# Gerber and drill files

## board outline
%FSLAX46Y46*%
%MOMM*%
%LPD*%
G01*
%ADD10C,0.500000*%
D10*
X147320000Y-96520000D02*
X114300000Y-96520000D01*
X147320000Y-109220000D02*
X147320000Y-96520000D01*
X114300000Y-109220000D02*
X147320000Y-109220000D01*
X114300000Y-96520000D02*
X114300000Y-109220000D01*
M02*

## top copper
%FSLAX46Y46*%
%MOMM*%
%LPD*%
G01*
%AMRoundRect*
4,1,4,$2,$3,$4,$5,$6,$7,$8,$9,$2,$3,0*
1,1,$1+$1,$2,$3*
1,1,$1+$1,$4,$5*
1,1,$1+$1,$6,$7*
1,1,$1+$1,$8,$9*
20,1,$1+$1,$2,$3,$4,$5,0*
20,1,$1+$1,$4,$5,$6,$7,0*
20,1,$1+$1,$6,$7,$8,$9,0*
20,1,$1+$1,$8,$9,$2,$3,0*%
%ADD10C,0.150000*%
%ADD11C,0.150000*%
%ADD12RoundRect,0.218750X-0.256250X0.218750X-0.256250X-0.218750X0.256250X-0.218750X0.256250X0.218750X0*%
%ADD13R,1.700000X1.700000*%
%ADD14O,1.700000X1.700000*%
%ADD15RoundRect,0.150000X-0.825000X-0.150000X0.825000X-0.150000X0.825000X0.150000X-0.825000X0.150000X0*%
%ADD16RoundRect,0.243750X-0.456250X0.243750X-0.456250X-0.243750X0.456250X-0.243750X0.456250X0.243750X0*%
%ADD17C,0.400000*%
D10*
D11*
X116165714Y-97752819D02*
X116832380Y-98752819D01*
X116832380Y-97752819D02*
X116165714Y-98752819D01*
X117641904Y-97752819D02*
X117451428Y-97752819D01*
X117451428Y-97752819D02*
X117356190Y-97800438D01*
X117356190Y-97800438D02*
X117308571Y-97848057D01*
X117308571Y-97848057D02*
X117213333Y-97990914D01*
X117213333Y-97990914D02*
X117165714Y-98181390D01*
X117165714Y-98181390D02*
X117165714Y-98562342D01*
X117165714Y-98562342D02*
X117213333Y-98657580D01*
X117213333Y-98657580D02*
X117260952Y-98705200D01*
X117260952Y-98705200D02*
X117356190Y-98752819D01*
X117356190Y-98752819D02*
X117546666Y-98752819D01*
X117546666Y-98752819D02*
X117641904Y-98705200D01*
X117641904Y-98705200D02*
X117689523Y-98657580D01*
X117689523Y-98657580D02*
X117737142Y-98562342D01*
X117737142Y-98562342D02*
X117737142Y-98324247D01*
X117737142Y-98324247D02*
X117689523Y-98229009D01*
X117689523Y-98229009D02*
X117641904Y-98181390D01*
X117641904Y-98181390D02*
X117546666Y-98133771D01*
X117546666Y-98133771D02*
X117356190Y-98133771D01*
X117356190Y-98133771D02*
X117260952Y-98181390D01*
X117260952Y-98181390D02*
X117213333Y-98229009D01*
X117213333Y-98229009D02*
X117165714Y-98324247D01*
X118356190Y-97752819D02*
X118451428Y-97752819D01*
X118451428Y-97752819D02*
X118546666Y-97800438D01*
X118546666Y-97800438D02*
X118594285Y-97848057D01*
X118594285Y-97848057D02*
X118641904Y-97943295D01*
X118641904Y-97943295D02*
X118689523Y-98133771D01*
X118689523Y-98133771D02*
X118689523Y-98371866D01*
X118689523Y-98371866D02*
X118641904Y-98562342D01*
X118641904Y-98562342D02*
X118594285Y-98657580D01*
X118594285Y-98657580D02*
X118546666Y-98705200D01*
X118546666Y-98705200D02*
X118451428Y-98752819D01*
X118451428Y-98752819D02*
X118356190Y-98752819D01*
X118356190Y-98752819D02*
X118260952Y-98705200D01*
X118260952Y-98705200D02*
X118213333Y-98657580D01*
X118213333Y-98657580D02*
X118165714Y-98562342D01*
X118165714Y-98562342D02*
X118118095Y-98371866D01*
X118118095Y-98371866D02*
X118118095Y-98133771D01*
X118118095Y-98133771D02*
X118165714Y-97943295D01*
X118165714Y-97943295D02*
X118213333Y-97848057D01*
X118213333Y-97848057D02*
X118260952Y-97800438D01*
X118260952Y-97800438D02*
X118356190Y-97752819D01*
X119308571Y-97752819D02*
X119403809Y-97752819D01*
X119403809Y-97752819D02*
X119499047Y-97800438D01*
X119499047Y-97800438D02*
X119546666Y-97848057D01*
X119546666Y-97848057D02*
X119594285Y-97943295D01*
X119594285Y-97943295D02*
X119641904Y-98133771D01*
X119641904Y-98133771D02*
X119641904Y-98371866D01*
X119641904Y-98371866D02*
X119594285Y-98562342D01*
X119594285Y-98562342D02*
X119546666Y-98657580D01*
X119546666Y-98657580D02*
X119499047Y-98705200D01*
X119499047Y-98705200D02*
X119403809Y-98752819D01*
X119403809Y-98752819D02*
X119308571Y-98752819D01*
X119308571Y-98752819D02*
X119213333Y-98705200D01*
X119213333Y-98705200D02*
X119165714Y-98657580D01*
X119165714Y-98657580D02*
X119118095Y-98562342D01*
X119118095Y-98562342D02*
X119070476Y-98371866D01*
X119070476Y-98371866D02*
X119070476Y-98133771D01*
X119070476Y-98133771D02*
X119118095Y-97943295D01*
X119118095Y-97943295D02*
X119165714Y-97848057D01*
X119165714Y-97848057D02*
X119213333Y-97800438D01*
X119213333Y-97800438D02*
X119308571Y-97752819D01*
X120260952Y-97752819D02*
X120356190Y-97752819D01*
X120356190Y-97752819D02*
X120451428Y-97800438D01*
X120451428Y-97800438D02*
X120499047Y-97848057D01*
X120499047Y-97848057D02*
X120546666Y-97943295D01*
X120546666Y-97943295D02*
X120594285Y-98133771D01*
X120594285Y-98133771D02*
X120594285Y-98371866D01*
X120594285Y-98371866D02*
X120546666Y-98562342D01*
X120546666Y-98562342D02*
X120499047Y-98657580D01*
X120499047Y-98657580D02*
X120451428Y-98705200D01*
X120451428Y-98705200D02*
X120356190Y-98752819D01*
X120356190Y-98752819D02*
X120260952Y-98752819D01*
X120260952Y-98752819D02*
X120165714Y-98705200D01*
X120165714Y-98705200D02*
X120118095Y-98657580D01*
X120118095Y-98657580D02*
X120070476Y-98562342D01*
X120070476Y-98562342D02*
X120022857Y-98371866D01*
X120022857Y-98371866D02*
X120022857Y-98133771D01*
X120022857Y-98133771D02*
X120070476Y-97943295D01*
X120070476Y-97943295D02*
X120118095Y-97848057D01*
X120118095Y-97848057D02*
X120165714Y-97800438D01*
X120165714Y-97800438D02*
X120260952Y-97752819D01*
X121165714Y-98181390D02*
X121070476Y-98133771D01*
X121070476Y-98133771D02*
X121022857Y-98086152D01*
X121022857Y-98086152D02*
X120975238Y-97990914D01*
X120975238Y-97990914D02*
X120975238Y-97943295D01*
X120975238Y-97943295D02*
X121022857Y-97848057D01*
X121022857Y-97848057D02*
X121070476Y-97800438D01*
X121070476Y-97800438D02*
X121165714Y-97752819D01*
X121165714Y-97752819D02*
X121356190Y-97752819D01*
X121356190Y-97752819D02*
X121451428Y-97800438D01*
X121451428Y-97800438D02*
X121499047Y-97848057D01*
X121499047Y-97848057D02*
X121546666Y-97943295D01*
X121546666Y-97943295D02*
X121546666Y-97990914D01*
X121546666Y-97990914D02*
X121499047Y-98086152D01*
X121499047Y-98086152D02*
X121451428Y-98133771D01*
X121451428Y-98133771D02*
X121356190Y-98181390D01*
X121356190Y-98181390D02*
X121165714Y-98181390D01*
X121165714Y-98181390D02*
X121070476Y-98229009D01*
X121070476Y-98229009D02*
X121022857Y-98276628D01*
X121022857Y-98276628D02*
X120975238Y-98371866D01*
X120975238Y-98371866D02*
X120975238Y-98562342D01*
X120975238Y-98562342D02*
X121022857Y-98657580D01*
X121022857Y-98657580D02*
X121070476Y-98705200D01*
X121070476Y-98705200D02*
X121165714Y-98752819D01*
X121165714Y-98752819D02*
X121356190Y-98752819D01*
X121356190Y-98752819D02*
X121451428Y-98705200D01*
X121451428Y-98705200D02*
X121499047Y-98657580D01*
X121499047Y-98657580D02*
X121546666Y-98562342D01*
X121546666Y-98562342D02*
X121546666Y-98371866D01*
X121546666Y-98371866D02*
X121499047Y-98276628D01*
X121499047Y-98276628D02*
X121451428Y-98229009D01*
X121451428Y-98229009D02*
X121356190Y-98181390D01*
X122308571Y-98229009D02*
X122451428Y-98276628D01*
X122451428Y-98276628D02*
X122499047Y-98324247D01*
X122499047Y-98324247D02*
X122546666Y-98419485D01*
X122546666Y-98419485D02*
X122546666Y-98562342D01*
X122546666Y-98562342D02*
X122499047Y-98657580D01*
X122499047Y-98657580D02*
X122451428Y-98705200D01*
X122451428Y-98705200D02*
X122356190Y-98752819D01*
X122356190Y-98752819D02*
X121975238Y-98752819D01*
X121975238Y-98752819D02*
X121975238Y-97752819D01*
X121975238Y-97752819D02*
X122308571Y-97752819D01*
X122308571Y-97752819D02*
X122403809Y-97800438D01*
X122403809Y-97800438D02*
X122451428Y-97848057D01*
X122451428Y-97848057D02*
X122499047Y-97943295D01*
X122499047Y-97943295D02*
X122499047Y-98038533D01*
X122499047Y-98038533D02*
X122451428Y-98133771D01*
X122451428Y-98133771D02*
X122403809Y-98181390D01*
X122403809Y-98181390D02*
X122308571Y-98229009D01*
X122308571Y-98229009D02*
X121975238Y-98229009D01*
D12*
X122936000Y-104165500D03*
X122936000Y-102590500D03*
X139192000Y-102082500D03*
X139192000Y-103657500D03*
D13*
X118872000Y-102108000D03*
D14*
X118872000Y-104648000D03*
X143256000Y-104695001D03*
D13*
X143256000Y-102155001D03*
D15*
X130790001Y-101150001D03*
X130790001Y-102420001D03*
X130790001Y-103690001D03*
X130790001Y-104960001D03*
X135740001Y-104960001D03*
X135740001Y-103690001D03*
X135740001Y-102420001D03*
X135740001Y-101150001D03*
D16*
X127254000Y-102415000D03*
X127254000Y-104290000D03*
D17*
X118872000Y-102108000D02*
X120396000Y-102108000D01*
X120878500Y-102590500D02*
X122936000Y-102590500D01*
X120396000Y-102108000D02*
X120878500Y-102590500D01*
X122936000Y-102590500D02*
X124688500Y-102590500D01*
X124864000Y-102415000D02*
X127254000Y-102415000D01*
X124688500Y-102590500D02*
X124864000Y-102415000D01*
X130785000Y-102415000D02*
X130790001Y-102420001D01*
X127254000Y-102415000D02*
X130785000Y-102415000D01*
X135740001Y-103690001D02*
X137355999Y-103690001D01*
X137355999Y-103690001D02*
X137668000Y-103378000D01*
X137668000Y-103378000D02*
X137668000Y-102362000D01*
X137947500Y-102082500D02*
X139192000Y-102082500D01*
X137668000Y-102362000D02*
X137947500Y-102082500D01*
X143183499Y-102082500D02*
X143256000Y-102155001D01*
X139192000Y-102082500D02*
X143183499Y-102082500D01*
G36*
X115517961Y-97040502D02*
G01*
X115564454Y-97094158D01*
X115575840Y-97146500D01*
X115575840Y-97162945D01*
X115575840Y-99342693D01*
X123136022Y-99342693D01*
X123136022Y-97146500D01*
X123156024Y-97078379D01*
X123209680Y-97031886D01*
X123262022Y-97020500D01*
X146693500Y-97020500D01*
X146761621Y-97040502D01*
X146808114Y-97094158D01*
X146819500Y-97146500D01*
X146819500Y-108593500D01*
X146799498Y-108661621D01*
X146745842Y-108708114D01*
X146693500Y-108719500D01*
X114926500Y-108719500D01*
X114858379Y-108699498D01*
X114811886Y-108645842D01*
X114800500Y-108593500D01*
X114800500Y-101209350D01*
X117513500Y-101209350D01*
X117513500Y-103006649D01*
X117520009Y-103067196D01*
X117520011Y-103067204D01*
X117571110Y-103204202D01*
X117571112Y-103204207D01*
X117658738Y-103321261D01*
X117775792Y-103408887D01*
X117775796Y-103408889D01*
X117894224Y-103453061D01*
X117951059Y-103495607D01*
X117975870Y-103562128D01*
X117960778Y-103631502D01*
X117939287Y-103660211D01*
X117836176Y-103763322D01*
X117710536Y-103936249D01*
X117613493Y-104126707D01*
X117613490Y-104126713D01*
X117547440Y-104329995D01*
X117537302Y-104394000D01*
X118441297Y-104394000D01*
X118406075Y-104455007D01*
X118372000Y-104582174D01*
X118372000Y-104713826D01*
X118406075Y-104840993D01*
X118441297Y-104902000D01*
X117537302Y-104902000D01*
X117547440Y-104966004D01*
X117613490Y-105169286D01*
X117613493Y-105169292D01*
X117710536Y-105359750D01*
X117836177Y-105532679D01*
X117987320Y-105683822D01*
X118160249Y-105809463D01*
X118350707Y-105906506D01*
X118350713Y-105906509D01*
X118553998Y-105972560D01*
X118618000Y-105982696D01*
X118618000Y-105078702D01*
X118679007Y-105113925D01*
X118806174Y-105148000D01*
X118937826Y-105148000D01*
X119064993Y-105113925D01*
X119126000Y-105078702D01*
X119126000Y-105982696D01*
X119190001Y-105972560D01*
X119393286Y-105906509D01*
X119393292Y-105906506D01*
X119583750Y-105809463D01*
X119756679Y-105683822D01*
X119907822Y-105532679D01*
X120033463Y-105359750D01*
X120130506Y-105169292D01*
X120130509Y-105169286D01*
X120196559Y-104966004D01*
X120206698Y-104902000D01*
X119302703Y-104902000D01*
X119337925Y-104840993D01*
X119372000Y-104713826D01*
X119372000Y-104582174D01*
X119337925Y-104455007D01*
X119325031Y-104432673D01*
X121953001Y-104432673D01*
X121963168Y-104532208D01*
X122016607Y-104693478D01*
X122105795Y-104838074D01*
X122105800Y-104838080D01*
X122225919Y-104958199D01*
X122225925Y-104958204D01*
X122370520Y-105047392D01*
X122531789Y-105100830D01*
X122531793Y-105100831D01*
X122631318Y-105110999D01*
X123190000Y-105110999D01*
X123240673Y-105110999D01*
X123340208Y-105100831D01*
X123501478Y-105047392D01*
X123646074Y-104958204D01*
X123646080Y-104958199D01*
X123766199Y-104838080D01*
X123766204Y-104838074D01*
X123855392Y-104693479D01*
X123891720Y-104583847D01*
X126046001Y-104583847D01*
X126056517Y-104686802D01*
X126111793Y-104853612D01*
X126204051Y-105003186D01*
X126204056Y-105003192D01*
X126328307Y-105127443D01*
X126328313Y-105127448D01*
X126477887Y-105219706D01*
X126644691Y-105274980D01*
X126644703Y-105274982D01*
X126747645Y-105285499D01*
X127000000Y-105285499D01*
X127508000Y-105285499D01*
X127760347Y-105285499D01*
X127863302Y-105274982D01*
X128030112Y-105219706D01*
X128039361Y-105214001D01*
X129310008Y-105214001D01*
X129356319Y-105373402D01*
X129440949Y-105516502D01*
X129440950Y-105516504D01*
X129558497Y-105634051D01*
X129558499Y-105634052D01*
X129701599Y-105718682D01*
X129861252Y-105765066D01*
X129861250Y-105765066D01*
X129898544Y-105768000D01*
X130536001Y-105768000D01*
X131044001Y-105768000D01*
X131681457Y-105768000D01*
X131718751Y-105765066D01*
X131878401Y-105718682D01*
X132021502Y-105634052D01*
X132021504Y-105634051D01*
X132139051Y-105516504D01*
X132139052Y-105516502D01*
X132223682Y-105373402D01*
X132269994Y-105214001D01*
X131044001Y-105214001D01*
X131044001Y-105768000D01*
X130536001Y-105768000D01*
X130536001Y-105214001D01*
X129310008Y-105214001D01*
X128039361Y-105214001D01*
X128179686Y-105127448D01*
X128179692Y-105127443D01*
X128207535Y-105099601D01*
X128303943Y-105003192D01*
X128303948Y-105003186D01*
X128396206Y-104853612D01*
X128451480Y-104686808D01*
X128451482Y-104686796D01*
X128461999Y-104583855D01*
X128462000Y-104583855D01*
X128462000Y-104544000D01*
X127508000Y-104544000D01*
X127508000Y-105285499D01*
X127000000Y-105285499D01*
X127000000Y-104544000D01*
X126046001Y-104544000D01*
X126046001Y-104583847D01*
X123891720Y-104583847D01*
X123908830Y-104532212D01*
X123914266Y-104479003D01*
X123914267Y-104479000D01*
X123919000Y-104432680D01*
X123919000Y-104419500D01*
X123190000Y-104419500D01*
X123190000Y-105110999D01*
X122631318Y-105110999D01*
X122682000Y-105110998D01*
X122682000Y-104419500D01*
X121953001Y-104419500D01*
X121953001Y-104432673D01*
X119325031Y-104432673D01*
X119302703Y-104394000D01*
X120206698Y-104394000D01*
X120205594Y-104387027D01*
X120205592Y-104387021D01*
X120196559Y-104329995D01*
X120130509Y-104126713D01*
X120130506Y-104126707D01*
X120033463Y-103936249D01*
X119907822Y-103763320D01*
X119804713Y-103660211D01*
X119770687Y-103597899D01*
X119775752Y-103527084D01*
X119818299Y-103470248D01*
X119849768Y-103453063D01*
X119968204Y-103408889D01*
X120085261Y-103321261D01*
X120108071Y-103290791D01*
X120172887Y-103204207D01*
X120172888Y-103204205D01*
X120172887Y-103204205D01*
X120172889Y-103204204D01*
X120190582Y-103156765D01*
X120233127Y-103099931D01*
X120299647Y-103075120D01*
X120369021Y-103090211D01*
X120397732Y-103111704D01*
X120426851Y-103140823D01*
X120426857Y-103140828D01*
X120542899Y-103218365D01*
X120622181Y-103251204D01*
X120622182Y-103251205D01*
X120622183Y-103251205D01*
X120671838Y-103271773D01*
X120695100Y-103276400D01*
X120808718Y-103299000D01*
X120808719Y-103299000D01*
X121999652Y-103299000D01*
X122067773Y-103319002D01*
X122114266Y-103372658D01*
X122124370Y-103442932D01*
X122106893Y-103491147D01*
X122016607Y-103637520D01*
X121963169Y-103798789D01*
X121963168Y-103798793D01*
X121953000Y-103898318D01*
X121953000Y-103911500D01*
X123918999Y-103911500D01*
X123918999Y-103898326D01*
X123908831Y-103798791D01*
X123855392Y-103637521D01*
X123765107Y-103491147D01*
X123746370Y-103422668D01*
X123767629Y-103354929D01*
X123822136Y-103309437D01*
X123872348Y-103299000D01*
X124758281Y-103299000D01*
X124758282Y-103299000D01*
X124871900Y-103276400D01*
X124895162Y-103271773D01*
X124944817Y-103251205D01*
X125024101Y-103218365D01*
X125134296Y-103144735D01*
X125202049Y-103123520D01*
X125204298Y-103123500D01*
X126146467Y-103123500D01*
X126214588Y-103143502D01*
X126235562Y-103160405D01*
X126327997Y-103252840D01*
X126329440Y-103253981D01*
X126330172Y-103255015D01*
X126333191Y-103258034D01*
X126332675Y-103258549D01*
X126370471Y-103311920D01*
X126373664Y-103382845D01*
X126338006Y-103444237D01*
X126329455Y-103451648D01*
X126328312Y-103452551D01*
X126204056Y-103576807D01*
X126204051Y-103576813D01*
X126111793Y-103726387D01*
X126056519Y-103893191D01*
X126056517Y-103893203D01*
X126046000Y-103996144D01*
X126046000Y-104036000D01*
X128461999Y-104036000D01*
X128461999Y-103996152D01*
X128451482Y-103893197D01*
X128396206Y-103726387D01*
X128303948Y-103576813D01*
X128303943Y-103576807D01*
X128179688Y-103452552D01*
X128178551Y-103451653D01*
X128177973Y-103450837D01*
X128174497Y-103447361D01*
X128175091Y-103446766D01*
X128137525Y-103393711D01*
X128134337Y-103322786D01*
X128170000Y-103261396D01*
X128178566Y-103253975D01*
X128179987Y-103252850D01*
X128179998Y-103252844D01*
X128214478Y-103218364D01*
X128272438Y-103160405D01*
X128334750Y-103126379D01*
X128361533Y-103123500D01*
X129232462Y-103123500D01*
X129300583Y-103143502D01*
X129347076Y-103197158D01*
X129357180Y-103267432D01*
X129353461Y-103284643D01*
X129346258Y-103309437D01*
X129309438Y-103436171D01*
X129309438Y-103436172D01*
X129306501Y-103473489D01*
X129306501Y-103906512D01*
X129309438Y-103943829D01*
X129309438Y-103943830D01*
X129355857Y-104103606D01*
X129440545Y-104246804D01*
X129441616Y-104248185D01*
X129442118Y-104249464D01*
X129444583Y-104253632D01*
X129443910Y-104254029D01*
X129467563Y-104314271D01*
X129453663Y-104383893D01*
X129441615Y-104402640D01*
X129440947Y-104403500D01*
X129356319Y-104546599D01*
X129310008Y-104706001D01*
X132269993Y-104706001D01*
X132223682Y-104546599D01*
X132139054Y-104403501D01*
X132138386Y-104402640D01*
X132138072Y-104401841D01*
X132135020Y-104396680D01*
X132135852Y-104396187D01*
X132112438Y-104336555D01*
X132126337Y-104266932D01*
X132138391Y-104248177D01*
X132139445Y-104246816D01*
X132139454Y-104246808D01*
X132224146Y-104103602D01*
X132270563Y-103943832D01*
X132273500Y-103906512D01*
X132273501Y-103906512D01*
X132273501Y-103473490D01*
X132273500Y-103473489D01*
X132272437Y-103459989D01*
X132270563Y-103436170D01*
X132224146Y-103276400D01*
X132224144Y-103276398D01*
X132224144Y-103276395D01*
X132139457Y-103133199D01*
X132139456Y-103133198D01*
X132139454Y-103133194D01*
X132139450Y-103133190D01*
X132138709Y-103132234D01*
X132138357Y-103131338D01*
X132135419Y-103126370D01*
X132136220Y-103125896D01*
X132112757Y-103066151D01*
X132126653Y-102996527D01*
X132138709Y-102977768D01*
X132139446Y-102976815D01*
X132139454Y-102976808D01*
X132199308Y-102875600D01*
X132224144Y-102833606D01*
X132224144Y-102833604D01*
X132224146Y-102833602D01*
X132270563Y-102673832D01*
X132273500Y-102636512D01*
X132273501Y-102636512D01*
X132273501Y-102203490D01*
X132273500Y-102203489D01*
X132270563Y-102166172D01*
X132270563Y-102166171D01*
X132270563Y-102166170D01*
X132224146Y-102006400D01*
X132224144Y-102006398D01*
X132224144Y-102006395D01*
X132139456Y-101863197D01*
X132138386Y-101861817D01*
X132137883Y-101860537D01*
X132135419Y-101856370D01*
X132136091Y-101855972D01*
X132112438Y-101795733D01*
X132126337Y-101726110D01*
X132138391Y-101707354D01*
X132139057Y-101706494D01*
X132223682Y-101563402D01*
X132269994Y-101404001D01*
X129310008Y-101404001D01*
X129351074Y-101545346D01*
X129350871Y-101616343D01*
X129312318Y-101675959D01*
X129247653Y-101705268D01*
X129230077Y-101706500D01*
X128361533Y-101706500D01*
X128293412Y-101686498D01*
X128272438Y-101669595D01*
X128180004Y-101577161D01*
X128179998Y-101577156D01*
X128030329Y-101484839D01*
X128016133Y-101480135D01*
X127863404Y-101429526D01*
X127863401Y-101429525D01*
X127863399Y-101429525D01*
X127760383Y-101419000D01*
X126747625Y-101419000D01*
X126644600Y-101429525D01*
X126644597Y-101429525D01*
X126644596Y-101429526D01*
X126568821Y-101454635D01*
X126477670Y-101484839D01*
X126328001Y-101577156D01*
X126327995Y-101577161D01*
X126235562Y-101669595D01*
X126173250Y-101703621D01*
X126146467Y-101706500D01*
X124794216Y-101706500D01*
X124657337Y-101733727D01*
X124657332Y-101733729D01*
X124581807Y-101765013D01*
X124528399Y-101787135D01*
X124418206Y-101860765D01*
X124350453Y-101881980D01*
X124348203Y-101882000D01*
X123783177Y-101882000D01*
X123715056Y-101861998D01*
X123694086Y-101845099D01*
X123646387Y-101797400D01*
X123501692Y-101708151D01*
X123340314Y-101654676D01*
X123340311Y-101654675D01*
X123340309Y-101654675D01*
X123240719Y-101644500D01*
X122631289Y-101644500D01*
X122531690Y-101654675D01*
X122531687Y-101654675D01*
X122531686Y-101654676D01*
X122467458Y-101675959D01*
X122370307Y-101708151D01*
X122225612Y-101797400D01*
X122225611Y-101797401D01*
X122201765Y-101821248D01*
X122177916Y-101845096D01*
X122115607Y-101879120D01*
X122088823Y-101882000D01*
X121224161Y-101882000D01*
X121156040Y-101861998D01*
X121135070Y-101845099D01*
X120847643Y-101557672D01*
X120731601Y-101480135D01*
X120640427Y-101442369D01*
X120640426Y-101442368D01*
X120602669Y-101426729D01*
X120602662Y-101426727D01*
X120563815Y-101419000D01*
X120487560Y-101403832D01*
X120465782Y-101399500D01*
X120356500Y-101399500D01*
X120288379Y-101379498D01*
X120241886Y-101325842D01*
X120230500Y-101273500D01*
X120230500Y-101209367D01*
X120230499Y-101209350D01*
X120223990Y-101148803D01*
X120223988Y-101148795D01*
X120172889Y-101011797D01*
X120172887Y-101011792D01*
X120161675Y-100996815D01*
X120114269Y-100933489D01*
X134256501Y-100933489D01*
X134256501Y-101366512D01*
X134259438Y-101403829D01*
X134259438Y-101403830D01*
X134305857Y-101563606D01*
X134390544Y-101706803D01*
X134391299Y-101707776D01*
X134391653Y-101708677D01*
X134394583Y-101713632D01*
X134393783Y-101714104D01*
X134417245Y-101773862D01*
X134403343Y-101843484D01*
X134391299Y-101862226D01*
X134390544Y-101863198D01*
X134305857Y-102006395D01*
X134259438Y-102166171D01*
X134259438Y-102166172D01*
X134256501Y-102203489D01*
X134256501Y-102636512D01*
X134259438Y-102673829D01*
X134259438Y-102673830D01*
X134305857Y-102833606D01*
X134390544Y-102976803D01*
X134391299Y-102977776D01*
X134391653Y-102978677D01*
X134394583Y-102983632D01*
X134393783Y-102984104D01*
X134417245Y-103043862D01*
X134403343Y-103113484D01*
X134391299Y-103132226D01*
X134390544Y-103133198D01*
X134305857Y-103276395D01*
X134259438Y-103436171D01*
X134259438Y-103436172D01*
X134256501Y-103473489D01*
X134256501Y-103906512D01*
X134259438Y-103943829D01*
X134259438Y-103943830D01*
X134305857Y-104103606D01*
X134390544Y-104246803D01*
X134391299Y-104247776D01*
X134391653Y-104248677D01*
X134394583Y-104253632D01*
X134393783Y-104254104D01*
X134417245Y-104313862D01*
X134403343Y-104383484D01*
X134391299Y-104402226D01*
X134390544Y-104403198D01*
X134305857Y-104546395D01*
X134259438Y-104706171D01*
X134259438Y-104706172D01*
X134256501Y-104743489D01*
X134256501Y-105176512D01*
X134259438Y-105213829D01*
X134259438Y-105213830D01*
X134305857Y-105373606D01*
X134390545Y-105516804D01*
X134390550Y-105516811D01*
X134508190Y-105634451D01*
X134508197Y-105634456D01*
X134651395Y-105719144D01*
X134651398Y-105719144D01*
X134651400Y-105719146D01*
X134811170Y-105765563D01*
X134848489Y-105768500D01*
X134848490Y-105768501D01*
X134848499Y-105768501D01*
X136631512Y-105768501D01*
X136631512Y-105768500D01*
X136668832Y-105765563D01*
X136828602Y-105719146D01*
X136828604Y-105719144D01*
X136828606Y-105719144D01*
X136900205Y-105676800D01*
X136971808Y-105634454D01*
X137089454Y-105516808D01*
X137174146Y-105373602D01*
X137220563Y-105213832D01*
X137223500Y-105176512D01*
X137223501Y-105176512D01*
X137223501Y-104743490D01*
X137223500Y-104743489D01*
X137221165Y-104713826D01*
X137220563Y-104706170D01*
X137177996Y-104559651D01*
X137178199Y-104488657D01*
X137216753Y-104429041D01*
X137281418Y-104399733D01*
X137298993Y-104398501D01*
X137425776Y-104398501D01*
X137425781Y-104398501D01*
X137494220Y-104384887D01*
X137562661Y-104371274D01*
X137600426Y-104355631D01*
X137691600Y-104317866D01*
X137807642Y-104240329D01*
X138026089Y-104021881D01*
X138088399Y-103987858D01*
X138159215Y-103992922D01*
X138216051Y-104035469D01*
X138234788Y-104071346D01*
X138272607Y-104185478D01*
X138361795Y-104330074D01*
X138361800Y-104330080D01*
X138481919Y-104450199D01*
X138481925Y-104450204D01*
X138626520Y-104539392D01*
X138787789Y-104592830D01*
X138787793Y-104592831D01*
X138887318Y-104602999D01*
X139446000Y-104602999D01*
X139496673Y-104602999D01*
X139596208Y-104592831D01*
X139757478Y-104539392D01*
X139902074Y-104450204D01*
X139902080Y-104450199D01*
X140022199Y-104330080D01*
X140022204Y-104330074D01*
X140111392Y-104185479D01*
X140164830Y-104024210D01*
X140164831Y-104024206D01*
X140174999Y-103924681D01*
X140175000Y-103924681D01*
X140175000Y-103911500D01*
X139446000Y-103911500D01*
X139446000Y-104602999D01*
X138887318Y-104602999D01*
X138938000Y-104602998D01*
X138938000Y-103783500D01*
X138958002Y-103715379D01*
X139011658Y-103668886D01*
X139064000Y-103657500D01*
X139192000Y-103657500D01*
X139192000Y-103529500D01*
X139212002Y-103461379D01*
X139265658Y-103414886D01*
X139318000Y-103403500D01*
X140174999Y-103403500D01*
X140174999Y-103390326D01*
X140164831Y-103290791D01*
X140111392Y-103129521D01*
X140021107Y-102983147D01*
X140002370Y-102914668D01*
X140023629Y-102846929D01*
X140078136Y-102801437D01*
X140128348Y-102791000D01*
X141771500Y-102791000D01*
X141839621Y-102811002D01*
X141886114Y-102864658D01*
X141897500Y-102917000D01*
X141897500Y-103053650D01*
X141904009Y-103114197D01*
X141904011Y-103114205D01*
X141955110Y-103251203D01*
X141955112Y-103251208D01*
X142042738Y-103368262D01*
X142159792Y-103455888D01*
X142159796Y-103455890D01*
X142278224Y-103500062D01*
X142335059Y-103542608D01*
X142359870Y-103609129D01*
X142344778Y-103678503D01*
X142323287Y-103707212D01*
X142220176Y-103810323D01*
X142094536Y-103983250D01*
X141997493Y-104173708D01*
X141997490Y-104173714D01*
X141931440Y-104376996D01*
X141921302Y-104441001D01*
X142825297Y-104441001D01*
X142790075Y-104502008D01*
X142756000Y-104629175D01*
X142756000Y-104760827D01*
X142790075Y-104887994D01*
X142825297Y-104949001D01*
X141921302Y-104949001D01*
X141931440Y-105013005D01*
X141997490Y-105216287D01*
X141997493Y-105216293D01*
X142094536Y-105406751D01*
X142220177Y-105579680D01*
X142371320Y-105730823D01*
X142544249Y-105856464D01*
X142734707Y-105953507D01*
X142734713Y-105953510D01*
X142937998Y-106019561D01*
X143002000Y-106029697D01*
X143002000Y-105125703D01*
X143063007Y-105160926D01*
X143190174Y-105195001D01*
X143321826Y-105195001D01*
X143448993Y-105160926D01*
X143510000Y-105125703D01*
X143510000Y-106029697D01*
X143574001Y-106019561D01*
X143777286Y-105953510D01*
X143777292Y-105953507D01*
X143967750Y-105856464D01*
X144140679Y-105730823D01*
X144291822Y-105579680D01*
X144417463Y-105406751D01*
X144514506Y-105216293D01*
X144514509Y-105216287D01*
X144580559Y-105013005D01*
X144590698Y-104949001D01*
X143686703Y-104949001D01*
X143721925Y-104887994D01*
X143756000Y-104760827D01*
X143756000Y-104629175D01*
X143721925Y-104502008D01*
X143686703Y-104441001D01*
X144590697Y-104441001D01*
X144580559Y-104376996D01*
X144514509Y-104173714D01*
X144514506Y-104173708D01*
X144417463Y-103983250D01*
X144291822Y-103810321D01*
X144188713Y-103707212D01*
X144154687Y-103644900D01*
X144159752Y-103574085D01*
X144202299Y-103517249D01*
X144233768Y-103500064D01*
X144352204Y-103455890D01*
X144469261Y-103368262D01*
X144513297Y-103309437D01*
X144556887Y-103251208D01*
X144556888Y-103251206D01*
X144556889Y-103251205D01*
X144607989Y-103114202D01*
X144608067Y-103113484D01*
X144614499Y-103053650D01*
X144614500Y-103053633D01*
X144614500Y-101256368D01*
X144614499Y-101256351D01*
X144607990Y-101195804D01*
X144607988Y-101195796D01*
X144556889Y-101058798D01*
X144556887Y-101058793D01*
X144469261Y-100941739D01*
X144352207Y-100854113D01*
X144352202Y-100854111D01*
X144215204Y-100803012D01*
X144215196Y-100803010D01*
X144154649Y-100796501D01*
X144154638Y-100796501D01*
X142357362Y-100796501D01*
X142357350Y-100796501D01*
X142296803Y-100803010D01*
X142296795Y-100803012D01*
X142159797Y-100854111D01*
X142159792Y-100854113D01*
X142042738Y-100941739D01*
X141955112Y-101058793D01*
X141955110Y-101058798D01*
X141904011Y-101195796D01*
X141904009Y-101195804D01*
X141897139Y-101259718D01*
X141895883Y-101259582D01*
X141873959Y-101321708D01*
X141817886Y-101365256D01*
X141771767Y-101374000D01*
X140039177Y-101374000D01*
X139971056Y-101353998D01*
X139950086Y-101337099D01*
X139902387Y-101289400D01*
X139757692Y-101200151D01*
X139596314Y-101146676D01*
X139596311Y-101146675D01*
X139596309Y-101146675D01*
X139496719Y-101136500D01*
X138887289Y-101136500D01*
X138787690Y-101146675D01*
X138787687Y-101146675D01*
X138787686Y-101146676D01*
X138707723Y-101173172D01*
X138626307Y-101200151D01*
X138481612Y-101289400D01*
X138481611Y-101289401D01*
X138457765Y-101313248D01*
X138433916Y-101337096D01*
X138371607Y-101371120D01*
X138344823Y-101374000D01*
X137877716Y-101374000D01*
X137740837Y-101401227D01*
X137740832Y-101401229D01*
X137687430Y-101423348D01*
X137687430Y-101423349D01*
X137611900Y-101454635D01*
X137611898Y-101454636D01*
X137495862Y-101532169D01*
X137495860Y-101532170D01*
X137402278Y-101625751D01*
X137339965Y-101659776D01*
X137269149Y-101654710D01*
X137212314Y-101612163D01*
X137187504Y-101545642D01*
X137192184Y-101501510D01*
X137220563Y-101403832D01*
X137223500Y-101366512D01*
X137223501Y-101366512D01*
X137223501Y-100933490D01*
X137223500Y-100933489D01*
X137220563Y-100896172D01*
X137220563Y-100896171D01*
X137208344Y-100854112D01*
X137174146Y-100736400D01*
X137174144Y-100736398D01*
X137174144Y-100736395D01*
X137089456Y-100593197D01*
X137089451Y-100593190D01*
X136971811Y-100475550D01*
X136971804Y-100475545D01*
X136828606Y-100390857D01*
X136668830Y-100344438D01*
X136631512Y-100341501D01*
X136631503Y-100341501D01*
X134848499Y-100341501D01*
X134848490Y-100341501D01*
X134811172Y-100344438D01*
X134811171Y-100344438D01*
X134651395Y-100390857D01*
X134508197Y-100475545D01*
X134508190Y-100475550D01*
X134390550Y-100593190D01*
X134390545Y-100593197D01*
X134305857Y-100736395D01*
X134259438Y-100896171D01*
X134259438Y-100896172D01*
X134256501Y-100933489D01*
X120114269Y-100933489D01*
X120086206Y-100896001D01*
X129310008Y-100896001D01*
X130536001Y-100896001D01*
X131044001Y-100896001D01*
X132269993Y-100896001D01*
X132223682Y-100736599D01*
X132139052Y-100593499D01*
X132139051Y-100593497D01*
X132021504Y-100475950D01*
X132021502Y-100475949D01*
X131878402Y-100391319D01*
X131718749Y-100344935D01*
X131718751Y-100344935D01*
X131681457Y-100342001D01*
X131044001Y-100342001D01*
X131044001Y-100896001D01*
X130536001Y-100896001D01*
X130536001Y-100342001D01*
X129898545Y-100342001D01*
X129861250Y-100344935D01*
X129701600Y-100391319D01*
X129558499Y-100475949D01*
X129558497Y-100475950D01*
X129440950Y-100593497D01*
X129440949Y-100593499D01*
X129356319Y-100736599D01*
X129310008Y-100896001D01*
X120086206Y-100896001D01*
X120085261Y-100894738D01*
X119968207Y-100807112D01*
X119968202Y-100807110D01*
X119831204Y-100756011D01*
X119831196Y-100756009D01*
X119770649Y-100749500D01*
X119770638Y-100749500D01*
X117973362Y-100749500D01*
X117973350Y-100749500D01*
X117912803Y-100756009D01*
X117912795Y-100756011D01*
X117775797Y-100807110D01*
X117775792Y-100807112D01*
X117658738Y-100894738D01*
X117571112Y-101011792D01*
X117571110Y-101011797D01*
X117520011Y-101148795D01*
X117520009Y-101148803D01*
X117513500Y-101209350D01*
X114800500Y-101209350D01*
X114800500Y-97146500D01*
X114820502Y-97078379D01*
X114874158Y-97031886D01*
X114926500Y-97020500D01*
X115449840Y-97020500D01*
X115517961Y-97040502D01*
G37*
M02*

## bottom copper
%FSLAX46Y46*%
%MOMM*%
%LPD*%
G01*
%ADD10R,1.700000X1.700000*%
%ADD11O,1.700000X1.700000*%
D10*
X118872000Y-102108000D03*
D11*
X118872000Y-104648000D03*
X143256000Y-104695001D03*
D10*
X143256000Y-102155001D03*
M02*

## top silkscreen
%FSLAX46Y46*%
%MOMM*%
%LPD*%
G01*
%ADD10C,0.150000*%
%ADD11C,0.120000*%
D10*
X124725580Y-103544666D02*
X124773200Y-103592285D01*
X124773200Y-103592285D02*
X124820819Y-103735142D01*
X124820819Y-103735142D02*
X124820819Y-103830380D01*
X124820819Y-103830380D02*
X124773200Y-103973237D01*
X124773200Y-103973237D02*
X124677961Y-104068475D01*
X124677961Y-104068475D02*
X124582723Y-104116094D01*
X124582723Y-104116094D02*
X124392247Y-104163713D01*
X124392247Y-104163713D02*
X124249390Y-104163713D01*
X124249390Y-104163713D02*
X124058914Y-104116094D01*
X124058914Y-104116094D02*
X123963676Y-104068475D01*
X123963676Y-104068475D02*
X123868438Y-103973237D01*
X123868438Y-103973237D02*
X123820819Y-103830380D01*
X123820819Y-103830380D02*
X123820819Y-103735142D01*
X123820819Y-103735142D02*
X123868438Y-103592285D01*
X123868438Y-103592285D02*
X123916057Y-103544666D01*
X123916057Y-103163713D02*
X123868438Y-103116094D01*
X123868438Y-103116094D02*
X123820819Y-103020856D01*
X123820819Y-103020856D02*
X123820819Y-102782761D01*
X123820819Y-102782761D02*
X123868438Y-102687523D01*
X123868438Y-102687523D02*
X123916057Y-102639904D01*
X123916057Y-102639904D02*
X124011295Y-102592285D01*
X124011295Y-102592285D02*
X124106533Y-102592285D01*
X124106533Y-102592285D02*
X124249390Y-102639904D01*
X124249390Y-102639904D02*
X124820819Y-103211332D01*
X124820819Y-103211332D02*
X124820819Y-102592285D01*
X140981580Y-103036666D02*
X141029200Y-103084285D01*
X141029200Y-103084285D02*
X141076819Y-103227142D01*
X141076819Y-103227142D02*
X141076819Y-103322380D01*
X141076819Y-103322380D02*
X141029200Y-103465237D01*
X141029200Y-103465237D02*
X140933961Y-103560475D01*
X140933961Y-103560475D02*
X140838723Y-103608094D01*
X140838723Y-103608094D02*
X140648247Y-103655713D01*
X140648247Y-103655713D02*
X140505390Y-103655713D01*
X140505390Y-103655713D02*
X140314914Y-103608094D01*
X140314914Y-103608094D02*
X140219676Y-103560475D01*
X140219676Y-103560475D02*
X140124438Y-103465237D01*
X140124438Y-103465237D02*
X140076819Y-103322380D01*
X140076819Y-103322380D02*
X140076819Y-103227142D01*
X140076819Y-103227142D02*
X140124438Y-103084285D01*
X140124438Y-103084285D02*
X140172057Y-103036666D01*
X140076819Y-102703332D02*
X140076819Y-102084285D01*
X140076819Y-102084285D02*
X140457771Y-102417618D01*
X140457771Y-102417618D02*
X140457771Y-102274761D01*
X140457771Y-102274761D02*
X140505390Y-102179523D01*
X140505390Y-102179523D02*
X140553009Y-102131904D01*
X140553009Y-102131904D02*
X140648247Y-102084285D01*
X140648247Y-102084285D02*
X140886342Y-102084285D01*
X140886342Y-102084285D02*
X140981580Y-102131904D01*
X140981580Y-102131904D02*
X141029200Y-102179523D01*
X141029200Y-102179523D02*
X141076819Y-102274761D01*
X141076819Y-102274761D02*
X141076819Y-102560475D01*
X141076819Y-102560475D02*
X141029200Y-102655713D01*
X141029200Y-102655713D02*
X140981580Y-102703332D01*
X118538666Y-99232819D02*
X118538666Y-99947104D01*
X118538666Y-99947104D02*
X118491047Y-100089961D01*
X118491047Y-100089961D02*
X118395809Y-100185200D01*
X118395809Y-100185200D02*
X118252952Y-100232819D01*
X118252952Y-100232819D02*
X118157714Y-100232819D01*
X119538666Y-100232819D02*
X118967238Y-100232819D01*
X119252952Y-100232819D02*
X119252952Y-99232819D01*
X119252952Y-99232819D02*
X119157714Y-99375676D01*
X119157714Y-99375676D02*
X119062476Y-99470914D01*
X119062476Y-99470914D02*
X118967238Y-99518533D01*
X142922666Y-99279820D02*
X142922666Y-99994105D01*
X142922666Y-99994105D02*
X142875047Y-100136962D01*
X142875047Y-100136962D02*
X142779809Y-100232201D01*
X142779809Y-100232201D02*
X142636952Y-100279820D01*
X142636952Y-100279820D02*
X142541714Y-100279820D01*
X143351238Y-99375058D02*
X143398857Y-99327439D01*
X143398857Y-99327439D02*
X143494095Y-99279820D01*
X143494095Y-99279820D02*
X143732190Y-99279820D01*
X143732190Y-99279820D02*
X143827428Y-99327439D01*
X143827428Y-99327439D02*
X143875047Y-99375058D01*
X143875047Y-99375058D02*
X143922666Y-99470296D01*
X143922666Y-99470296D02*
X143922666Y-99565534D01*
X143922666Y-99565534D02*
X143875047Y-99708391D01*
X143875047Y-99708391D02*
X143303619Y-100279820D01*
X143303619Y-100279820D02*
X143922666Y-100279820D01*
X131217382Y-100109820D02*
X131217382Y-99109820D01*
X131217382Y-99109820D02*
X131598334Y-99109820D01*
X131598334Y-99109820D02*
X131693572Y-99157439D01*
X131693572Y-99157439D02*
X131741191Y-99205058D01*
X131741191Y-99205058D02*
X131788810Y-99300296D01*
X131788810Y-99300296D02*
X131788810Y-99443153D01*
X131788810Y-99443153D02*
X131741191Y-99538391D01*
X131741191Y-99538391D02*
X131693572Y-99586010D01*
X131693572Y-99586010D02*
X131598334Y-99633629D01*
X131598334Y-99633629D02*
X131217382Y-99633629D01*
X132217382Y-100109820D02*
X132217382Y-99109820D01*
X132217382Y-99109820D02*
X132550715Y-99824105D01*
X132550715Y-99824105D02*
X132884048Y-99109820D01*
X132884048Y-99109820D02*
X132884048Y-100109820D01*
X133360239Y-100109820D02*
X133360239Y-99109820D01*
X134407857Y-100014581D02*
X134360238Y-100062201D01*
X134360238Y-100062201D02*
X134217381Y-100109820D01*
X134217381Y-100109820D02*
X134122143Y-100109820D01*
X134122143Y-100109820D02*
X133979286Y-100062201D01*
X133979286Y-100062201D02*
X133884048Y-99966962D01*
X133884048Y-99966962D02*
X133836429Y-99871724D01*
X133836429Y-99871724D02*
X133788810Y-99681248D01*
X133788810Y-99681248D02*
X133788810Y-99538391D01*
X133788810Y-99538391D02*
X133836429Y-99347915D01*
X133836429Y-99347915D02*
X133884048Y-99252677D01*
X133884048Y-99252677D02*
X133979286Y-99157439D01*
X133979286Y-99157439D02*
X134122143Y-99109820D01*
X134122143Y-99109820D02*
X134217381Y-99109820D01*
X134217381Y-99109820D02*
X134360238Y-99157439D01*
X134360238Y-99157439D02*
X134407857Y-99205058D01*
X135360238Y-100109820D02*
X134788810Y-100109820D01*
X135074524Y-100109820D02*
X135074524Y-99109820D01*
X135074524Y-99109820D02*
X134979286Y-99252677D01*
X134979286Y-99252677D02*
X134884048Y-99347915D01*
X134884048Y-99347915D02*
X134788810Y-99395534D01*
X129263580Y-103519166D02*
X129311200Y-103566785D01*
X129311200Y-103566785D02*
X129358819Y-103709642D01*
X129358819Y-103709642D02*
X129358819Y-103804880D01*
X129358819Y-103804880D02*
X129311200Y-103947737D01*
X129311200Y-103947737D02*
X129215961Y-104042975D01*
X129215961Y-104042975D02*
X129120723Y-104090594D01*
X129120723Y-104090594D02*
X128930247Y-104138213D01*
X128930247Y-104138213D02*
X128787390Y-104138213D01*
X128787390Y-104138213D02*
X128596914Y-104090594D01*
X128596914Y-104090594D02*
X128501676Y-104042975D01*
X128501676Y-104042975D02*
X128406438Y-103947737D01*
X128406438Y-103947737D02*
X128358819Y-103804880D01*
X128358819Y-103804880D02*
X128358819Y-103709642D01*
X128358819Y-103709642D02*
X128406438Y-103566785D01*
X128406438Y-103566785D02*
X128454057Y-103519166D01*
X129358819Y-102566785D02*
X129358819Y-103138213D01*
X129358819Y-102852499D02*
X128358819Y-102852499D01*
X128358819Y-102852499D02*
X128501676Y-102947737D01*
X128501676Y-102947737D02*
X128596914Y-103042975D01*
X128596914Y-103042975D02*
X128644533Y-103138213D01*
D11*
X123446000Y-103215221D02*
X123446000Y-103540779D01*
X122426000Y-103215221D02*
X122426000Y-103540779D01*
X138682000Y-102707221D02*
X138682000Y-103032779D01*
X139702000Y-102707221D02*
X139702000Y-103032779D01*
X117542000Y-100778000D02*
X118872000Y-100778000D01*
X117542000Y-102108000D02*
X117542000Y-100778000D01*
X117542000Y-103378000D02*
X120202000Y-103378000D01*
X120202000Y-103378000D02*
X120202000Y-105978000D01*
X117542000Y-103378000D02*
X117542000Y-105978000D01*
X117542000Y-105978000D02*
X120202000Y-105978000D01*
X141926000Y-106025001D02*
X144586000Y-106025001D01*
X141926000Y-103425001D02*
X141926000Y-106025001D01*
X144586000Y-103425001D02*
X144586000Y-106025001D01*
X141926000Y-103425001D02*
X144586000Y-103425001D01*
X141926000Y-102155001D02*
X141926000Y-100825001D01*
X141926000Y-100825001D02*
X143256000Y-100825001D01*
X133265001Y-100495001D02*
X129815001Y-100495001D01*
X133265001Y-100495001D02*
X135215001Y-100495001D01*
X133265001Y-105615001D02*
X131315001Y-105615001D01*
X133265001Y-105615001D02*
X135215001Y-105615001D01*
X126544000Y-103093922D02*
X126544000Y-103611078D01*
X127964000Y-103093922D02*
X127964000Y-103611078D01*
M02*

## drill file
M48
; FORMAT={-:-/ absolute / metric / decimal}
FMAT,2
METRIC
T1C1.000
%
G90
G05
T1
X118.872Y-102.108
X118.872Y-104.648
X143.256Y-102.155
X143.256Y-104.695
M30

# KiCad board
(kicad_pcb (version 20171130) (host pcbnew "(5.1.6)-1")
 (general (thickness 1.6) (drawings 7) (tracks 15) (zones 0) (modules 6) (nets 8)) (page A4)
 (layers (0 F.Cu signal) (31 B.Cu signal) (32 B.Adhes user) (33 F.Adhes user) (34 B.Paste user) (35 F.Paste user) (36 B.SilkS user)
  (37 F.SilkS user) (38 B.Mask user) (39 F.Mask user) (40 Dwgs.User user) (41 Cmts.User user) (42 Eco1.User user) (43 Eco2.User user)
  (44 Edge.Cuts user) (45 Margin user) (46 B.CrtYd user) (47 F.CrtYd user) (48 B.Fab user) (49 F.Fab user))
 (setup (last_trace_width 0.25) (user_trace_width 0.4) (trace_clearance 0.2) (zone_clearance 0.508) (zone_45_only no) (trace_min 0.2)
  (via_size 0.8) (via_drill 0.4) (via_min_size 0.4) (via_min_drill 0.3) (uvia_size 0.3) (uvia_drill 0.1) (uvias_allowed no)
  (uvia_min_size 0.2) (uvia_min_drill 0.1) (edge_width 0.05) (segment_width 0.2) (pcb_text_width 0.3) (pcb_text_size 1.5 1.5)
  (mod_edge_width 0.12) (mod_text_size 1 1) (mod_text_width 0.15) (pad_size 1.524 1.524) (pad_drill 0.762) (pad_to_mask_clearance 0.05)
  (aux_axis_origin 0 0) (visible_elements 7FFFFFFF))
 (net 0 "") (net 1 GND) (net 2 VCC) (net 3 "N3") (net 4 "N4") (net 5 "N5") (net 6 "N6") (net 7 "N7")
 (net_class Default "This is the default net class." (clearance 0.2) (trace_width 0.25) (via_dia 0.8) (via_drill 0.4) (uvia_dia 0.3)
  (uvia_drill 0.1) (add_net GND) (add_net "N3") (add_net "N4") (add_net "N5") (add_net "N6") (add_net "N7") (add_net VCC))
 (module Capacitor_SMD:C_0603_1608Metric (layer F.Cu) (at 122.936 103.378 270)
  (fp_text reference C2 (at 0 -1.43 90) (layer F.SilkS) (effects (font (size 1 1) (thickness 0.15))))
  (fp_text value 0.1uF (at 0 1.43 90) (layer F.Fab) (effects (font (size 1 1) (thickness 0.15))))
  (fp_line (start -0.162779 -0.51) (end 0.162779 -0.51) (layer F.SilkS) (width 0.12))
  (fp_line (start -0.162779 0.51) (end 0.162779 0.51) (layer F.SilkS) (width 0.12))
  (pad 2 smd roundrect (at 0.7875 0 270) (size 0.875 0.95) (layers F.Cu F.Paste F.Mask) (roundrect_rratio 0.25) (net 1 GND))
  (pad 1 smd roundrect (at -0.7875 0 270) (size 0.875 0.95) (layers F.Cu F.Paste F.Mask) (roundrect_rratio 0.25) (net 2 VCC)))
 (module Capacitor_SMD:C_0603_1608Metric (layer F.Cu) (at 139.192 102.87 270)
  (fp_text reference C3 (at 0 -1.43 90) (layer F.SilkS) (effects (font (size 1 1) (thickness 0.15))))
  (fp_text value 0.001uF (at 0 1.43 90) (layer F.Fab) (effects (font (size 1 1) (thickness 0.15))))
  (fp_line (start -0.162779 0.51) (end 0.162779 0.51) (layer F.SilkS) (width 0.12))
  (fp_line (start -0.162779 -0.51) (end 0.162779 -0.51) (layer F.SilkS) (width 0.12))
  (pad 1 smd roundrect (at -0.7875 0 270) (size 0.875 0.95) (layers F.Cu F.Paste F.Mask) (roundrect_rratio 0.25) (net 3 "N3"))
  (pad 2 smd roundrect (at 0.7875 0 270) (size 0.875 0.95) (layers F.Cu F.Paste F.Mask) (roundrect_rratio 0.25) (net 1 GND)))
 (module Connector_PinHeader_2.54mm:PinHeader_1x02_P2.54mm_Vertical (layer F.Cu) (at 118.872 102.108)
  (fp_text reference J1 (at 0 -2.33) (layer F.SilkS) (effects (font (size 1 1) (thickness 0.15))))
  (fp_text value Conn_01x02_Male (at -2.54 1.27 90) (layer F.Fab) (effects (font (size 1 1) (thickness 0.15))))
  (fp_line (start -1.33 -1.33) (end 0 -1.33) (layer F.SilkS) (width 0.12))
  (fp_line (start -1.33 0) (end -1.33 -1.33) (layer F.SilkS) (width 0.12))
  (fp_line (start -1.33 1.27) (end 1.33 1.27) (layer F.SilkS) (width 0.12))
  (fp_line (start 1.33 1.27) (end 1.33 3.87) (layer F.SilkS) (width 0.12))
  (fp_line (start -1.33 1.27) (end -1.33 3.87) (layer F.SilkS) (width 0.12))
  (fp_line (start -1.33 3.87) (end 1.33 3.87) (layer F.SilkS) (width 0.12))
  (pad 1 thru_hole rect (at 0 0) (size 1.7 1.7) (drill 1) (layers *.Cu *.Mask) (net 2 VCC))
  (pad 2 thru_hole oval (at 0 2.54) (size 1.7 1.7) (drill 1) (layers *.Cu *.Mask) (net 1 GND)))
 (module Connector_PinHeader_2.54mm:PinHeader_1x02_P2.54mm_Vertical (layer F.Cu) (at 143.256 102.155001)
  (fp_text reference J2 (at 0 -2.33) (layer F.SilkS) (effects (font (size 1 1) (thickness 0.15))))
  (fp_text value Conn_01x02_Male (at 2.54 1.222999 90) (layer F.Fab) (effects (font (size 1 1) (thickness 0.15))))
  (fp_line (start -1.33 3.87) (end 1.33 3.87) (layer F.SilkS) (width 0.12))
  (fp_line (start -1.33 1.27) (end -1.33 3.87) (layer F.SilkS) (width 0.12))
  (fp_line (start 1.33 1.27) (end 1.33 3.87) (layer F.SilkS) (width 0.12))
  (fp_line (start -1.33 1.27) (end 1.33 1.27) (layer F.SilkS) (width 0.12))
  (fp_line (start -1.33 0) (end -1.33 -1.33) (layer F.SilkS) (width 0.12))
  (fp_line (start -1.33 -1.33) (end 0 -1.33) (layer F.SilkS) (width 0.12))
  (pad 2 thru_hole oval (at 0 2.54) (size 1.7 1.7) (drill 1) (layers *.Cu *.Mask) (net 1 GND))
  (pad 1 thru_hole rect (at 0 0) (size 1.7 1.7) (drill 1) (layers *.Cu *.Mask) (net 3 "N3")))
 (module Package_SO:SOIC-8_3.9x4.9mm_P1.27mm (layer F.Cu) (at 133.265001 103.055001)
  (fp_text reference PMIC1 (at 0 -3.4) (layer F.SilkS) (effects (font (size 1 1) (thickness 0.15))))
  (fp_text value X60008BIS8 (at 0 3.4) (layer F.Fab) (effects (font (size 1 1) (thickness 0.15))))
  (fp_line (start 0 -2.56) (end -3.45 -2.56) (layer F.SilkS) (width 0.12))
  (fp_line (start 0 -2.56) (end 1.95 -2.56) (layer F.SilkS) (width 0.12))
  (fp_line (start 0 2.56) (end -1.95 2.56) (layer F.SilkS) (width 0.12))
  (fp_line (start 0 2.56) (end 1.95 2.56) (layer F.SilkS) (width 0.12))
  (pad 1 smd roundrect (at -2.475 -1.905) (size 1.95 0.6) (layers F.Cu F.Paste F.Mask) (roundrect_rratio 0.25) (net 1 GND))
  (pad 2 smd roundrect (at -2.475 -0.635) (size 1.95 0.6) (layers F.Cu F.Paste F.Mask) (roundrect_rratio 0.25) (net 2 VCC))
  (pad 3 smd roundrect (at -2.475 0.635) (size 1.95 0.6) (layers F.Cu F.Paste F.Mask) (roundrect_rratio 0.25) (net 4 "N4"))
  (pad 4 smd roundrect (at -2.475 1.905) (size 1.95 0.6) (layers F.Cu F.Paste F.Mask) (roundrect_rratio 0.25) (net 1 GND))
  (pad 5 smd roundrect (at 2.475 1.905) (size 1.95 0.6) (layers F.Cu F.Paste F.Mask) (roundrect_rratio 0.25) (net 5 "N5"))
  (pad 6 smd roundrect (at 2.475 0.635) (size 1.95 0.6) (layers F.Cu F.Paste F.Mask) (roundrect_rratio 0.25) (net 3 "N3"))
  (pad 7 smd roundrect (at 2.475 -0.635) (size 1.95 0.6) (layers F.Cu F.Paste F.Mask) (roundrect_rratio 0.25) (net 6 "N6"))
  (pad 8 smd roundrect (at 2.475 -1.905) (size 1.95 0.6) (layers F.Cu F.Paste F.Mask) (roundrect_rratio 0.25) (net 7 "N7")))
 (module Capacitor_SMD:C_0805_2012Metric (layer F.Cu) (at 127.254 103.3525 270)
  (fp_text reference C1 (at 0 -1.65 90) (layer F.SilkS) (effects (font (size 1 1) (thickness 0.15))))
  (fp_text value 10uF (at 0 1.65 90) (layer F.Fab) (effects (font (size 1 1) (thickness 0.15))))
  (fp_line (start -0.258578 0.71) (end 0.258578 0.71) (layer F.SilkS) (width 0.12))
  (fp_line (start -0.258578 -0.71) (end 0.258578 -0.71) (layer F.SilkS) (width 0.12))
  (pad 1 smd roundrect (at -0.9375 0 270) (size 0.975 1.4) (layers F.Cu F.Paste F.Mask) (roundrect_rratio 0.25) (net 2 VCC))
  (pad 2 smd roundrect (at 0.9375 0 270) (size 0.975 1.4) (layers F.Cu F.Paste F.Mask) (roundrect_rratio 0.25) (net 1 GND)))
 (gr_line (start 147.32 96.52) (end 114.3 96.52) (layer Edge.Cuts) (width 0.5))
 (gr_line (start 147.32 109.22) (end 147.32 96.52) (layer Edge.Cuts) (width 0.5))
 (gr_line (start 114.3 109.22) (end 147.32 109.22) (layer Edge.Cuts) (width 0.5))
 (gr_line (start 114.3 96.52) (end 114.3 109.22) (layer Edge.Cuts) (width 0.5))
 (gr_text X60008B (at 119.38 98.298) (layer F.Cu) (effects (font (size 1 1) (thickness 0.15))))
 (segment (start 118.872 102.108) (end 120.396 102.108) (width 0.4) (layer F.Cu) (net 2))
 (segment (start 120.8785 102.5905) (end 122.936 102.5905) (width 0.4) (layer F.Cu) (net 2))
 (segment (start 120.396 102.108) (end 120.8785 102.5905) (width 0.4) (layer F.Cu) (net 2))
 (segment (start 122.936 102.5905) (end 124.6885 102.5905) (width 0.4) (layer F.Cu) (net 2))
 (segment (start 124.864 102.415) (end 127.254 102.415) (width 0.4) (layer F.Cu) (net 2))
 (segment (start 124.6885 102.5905) (end 124.864 102.415) (width 0.4) (layer F.Cu) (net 2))
 (segment (start 130.785 102.415) (end 130.790001 102.420001) (width 0.4) (layer F.Cu) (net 2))
 (segment (start 127.254 102.415) (end 130.785 102.415) (width 0.4) (layer F.Cu) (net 2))
 (segment (start 135.740001 103.690001) (end 137.355999 103.690001) (width 0.4) (layer F.Cu) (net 3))
 (segment (start 137.355999 103.690001) (end 137.668 103.378) (width 0.4) (layer F.Cu) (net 3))
 (segment (start 137.668 103.378) (end 137.668 102.362) (width 0.4) (layer F.Cu) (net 3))
 (segment (start 137.9475 102.0825) (end 139.192 102.0825) (width 0.4) (layer F.Cu) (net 3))
 (segment (start 137.668 102.362) (end 137.9475 102.0825) (width 0.4) (layer F.Cu) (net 3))
 (segment (start 143.183499 102.0825) (end 143.256 102.155001) (width 0.4) (layer F.Cu) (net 3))
 (segment (start 139.192 102.0825) (end 143.183499 102.0825) (width 0.4) (layer F.Cu) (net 3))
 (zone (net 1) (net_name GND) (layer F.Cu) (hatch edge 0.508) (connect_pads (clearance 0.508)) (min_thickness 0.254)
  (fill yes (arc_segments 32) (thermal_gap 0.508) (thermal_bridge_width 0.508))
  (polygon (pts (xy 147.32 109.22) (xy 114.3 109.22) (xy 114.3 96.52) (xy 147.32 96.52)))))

